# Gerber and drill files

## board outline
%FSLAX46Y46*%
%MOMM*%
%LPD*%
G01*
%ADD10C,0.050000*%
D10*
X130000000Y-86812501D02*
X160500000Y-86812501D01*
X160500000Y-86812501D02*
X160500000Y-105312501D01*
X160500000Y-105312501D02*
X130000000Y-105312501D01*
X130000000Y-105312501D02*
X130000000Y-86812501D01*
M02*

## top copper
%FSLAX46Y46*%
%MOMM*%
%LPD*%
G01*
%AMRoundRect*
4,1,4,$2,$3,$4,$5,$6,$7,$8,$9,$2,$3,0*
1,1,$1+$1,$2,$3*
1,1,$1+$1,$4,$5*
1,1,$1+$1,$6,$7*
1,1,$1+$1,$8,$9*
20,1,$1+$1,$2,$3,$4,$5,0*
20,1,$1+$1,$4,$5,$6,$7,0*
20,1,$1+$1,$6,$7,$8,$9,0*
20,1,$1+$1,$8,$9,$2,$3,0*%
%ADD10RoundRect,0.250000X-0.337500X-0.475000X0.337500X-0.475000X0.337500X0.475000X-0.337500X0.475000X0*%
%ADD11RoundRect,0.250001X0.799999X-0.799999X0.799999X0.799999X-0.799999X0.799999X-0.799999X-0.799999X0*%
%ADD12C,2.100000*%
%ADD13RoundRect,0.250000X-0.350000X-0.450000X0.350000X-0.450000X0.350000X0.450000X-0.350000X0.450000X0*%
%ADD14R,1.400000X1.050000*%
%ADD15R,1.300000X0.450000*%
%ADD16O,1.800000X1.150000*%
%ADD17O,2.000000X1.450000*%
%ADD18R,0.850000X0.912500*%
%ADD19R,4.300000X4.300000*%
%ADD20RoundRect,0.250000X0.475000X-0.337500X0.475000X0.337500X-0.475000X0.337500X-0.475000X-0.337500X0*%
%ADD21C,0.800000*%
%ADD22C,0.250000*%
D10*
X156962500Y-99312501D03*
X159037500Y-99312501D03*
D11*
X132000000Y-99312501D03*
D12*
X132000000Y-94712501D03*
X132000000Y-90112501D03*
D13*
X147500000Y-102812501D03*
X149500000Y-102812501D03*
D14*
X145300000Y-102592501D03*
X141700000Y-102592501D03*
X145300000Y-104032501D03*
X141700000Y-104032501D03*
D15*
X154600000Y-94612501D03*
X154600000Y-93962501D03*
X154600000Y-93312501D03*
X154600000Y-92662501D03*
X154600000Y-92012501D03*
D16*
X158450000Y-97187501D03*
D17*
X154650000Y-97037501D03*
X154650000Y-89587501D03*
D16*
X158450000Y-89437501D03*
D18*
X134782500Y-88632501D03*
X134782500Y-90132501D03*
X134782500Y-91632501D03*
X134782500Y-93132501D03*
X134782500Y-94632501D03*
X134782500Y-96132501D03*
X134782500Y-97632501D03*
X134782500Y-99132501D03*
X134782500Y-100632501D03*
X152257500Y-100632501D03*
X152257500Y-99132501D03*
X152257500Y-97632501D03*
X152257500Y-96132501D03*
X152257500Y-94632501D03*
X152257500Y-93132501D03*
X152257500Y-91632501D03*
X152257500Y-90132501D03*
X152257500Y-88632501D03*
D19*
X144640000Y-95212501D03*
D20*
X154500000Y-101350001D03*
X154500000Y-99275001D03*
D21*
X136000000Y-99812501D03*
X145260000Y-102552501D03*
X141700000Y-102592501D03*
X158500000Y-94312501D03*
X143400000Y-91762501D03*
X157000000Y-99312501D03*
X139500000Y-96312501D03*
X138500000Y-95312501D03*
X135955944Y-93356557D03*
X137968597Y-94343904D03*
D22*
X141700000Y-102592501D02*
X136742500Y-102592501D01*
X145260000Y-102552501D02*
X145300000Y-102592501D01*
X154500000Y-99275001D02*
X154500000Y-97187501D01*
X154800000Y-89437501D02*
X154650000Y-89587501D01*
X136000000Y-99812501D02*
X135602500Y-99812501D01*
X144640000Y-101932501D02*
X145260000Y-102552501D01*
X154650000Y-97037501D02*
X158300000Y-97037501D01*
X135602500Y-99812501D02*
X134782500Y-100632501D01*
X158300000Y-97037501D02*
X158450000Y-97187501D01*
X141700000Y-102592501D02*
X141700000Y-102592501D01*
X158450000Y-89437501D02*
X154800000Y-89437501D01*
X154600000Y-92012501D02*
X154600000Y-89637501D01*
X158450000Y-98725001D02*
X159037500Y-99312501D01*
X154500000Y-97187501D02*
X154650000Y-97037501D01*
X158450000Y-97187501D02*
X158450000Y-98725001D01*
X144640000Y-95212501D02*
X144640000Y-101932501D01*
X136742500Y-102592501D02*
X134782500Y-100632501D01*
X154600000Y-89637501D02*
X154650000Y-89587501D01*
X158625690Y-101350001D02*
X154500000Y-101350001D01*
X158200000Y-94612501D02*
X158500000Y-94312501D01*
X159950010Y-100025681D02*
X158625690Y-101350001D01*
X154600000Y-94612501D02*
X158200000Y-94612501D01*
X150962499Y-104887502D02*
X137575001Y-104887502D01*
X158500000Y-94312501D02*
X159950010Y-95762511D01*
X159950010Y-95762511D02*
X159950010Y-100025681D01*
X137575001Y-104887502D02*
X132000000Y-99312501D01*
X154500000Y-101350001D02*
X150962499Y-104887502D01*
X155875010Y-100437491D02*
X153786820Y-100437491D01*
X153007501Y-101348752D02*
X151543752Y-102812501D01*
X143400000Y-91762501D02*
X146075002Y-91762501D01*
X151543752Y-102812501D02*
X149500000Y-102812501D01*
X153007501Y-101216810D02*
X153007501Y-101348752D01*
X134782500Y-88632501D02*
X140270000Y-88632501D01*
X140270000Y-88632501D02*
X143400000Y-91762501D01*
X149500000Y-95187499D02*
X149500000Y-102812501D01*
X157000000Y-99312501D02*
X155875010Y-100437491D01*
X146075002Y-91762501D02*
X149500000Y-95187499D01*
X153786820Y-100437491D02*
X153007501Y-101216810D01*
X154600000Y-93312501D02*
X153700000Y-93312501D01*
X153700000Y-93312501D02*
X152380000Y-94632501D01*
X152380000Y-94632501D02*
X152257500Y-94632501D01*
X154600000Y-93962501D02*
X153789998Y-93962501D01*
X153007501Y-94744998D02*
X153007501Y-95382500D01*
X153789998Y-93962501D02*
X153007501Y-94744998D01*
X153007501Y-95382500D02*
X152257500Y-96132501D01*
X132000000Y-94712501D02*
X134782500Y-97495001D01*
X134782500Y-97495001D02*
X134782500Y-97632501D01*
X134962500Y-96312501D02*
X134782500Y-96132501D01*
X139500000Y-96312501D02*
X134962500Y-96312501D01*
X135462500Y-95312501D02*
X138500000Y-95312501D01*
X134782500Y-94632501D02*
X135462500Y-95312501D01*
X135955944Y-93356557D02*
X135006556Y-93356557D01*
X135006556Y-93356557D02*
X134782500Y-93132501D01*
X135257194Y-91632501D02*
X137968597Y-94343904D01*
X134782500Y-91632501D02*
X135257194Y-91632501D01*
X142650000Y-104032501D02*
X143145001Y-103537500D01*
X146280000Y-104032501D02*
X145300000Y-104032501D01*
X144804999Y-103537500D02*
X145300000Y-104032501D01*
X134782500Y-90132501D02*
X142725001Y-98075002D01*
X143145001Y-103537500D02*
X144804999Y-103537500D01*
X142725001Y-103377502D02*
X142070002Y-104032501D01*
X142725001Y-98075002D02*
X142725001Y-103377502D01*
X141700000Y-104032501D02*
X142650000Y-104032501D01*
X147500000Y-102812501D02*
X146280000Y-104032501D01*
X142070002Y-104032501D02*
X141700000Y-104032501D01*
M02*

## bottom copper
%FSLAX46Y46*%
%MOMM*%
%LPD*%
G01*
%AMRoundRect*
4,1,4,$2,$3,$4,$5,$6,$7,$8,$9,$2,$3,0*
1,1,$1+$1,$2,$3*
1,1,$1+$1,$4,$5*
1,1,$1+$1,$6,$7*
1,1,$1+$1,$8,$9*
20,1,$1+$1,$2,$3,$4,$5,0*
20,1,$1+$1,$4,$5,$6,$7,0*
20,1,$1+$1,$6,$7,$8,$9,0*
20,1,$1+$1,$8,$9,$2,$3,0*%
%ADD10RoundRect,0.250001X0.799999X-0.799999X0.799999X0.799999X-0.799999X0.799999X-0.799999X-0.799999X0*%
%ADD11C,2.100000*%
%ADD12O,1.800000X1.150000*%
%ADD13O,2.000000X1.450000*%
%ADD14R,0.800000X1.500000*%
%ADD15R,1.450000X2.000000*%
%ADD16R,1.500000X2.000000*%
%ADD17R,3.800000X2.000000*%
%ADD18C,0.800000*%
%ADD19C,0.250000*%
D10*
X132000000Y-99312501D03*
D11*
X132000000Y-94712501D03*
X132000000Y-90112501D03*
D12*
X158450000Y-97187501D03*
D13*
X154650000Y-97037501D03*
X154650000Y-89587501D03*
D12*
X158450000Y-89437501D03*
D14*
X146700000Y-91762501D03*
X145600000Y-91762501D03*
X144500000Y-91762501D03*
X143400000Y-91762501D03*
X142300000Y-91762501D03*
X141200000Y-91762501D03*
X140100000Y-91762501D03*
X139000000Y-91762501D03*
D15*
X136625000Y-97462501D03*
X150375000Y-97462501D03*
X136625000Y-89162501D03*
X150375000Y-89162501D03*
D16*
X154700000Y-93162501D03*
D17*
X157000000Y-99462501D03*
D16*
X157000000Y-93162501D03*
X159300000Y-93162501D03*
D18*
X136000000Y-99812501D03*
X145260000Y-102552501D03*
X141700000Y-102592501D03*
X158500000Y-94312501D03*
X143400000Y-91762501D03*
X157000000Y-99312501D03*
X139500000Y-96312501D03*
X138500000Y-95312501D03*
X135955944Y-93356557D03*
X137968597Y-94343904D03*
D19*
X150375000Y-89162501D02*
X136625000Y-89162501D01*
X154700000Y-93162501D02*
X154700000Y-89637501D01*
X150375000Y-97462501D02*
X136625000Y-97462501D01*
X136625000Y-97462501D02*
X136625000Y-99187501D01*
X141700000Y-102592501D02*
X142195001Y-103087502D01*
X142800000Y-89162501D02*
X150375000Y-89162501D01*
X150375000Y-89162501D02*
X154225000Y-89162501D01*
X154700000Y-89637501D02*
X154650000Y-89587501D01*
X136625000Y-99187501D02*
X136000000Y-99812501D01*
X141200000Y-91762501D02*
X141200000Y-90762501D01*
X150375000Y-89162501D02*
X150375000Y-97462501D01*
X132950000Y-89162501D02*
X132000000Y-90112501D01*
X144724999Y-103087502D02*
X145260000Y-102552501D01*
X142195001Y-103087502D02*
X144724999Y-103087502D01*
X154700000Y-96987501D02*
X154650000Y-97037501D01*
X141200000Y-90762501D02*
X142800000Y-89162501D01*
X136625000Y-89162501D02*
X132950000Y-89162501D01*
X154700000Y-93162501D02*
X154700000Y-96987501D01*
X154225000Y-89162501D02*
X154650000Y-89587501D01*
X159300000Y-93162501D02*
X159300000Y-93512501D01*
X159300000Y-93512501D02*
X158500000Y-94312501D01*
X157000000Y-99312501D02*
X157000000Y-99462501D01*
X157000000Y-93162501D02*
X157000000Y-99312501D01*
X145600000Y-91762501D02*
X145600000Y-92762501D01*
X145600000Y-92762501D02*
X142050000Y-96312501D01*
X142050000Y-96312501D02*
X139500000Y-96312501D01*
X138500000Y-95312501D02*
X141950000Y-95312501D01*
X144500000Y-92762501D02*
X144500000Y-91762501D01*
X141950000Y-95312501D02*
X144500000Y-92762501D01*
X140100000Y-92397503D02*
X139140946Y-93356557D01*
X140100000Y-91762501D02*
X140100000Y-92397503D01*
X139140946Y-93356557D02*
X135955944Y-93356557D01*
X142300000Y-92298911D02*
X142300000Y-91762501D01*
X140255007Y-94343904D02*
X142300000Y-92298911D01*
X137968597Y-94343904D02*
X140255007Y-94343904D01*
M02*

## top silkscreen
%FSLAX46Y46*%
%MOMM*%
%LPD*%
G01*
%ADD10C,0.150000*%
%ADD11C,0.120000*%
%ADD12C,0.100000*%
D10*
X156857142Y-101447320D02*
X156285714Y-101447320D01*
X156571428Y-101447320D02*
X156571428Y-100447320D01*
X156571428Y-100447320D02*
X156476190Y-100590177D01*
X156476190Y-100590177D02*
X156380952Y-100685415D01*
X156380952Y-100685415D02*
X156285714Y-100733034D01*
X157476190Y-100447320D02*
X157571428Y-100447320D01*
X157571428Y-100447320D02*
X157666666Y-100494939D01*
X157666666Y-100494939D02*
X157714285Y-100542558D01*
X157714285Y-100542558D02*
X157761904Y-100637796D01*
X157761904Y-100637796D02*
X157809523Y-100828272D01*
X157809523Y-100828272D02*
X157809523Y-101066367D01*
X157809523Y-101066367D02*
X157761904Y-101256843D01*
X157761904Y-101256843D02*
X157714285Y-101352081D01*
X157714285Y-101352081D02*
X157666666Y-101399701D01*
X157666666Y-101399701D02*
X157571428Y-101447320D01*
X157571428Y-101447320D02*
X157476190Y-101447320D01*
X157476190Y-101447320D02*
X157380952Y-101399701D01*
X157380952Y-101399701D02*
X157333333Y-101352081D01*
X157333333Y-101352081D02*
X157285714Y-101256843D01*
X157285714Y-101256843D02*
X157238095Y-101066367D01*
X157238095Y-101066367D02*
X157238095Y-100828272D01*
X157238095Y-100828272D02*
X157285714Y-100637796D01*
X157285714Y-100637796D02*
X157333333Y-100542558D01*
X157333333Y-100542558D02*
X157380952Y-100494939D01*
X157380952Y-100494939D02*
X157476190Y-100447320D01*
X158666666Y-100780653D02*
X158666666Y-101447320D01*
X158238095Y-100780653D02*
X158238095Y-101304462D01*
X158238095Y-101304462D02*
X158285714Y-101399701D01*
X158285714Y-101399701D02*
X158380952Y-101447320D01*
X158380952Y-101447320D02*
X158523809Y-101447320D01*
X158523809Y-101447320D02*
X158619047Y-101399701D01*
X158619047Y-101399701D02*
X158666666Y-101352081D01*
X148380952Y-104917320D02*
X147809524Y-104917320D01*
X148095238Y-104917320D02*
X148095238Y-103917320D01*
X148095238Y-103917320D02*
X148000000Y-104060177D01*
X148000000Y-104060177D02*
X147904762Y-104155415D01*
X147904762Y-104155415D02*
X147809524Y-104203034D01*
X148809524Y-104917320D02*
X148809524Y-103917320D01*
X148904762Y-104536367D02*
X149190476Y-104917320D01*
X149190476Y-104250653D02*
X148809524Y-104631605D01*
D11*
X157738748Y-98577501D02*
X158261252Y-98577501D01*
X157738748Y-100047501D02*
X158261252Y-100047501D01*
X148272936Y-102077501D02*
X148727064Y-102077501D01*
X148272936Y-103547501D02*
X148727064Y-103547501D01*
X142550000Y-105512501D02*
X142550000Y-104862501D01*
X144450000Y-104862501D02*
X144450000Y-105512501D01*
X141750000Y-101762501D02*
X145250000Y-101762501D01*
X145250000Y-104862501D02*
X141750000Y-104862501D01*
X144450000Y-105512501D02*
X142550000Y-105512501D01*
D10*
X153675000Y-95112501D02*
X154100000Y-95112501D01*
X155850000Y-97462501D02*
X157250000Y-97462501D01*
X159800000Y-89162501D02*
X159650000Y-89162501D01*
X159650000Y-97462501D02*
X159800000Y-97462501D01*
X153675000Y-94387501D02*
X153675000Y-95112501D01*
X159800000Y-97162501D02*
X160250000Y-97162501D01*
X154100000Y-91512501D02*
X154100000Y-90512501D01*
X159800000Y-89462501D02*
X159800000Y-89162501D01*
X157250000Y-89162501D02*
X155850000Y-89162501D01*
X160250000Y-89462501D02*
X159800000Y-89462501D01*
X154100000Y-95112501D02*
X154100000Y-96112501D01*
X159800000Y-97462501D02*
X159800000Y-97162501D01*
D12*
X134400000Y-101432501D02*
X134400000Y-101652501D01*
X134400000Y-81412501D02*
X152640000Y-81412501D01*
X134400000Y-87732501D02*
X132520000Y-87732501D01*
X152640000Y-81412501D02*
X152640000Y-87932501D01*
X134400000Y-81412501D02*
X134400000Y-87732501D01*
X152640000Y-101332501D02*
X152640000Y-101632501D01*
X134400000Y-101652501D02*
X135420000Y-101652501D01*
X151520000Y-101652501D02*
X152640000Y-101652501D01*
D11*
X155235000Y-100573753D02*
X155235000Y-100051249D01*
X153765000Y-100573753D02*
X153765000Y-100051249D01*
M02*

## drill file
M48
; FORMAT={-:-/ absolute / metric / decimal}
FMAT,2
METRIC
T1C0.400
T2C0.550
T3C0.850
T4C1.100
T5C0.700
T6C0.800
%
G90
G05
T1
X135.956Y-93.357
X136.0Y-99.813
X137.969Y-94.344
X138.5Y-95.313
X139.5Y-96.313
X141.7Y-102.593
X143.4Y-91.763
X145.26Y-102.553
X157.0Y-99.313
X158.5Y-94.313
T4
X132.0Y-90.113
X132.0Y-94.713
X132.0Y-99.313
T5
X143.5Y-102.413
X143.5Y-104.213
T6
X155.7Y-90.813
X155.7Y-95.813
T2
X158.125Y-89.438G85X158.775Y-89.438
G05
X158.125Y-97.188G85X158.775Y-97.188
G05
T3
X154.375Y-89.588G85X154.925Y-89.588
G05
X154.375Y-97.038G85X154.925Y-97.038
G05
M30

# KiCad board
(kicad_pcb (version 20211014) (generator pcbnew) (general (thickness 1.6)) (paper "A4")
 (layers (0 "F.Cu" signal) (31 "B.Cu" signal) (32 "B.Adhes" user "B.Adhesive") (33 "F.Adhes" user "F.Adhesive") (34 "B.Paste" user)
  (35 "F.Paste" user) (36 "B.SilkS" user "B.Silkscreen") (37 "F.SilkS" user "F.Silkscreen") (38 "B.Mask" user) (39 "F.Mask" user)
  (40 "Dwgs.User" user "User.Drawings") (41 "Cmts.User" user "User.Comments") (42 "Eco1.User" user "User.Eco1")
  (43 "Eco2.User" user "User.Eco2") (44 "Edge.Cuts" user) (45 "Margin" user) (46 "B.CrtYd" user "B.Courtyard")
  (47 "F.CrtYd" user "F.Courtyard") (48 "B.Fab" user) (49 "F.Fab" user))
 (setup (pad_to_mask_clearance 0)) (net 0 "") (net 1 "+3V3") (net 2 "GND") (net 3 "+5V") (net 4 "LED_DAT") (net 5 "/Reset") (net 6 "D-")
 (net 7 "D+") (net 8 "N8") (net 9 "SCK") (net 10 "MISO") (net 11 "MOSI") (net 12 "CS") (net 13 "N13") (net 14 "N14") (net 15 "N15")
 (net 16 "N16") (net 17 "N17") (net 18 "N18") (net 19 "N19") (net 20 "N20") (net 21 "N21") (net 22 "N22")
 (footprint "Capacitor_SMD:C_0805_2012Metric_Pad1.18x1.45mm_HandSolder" (layer "F.Cu") (at 158 99.312501)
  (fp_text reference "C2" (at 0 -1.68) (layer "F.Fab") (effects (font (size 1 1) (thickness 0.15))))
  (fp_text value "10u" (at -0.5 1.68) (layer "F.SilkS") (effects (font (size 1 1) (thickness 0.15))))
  (fp_line (start -0.261252 -0.735) (end 0.261252 -0.735) (layer "F.SilkS") (width 0.12))
  (fp_line (start -0.261252 0.735) (end 0.261252 0.735) (layer "F.SilkS") (width 0.12))
  (pad "1" smd roundrect locked (at -1.0375 0) (size 1.175 1.45) (layers "F.Cu" "F.Paste" "F.Mask") (roundrect_rratio 0.2127659574)
   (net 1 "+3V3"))
  (pad "2" smd roundrect locked (at 1.0375 0) (size 1.175 1.45) (layers "F.Cu" "F.Paste" "F.Mask") (roundrect_rratio 0.2127659574)
   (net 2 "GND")))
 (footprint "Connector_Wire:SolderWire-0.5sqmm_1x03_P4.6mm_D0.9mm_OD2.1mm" (layer "F.Cu") (at 132 99.312501 90)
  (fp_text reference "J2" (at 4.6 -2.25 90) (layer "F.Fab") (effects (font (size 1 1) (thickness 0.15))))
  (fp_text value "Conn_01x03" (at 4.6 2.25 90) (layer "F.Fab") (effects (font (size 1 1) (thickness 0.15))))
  (pad "1" thru_hole roundrect locked (at 0 0 90) (size 2.1 2.1) (drill 1.1) (layers *.Cu *.Mask) (roundrect_rratio 0.1190480952)
   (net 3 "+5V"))
  (pad "2" thru_hole circle locked (at 4.6 0 90) (size 2.1 2.1) (drill 1.1) (layers *.Cu *.Mask) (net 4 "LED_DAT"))
  (pad "3" thru_hole circle locked (at 9.2 0 90) (size 2.1 2.1) (drill 1.1) (layers *.Cu *.Mask) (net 2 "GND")))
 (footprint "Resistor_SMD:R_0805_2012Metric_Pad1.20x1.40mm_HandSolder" (layer "F.Cu") (at 148.5 102.812501)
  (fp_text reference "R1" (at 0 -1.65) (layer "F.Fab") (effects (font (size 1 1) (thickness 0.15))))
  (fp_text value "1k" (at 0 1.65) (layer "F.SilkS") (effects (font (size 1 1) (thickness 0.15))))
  (fp_line (start -0.227064 -0.735) (end 0.227064 -0.735) (layer "F.SilkS") (width 0.12))
  (fp_line (start -0.227064 0.735) (end 0.227064 0.735) (layer "F.SilkS") (width 0.12))
  (pad "1" smd roundrect locked (at -1 0) (size 1.2 1.4) (layers "F.Cu" "F.Paste" "F.Mask") (roundrect_rratio 0.2083333333) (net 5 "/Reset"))
  (pad "2" smd roundrect locked (at 1 0) (size 1.2 1.4) (layers "F.Cu" "F.Paste" "F.Mask") (roundrect_rratio 0.2083333333) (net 1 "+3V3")))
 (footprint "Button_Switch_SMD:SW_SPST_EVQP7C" (layer "F.Cu") (at 143.5 103.312501)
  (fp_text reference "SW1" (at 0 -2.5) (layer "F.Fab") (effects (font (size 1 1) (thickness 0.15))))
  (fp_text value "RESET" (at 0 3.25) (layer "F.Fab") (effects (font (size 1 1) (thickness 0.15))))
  (fp_line (start -0.95 2.2) (end -0.95 1.55) (layer "F.SilkS") (width 0.12))
  (fp_line (start 0.95 1.55) (end 0.95 2.2) (layer "F.SilkS") (width 0.12))
  (fp_line (start -1.75 -1.55) (end 1.75 -1.55) (layer "F.SilkS") (width 0.12))
  (fp_line (start 1.75 1.55) (end -1.75 1.55) (layer "F.SilkS") (width 0.12))
  (fp_line (start 0.95 2.2) (end -0.95 2.2) (layer "F.SilkS") (width 0.12))
  (pad "" np_thru_hole circle locked (at 0 0.9) (size 0.7 0.7) (drill 0.7) (layers *.Cu *.Mask))
  (pad "" np_thru_hole circle locked (at 0 -0.9) (size 0.7 0.7) (drill 0.7) (layers *.Cu *.Mask))
  (pad "1" smd rect locked (at 1.8 -0.72) (size 1.4 1.05) (layers "F.Cu" "F.Paste" "F.Mask") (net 2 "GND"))
  (pad "1" smd rect locked (at -1.8 -0.72) (size 1.4 1.05) (layers "F.Cu" "F.Paste" "F.Mask") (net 2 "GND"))
  (pad "2" smd rect locked (at 1.8 0.72) (size 1.4 1.05) (layers "F.Cu" "F.Paste" "F.Mask") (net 5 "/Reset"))
  (pad "2" smd rect locked (at -1.8 0.72) (size 1.4 1.05) (layers "F.Cu" "F.Paste" "F.Mask") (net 5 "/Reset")))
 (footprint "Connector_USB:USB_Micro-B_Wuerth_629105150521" (layer "F.Cu") (at 156.5 93.312501 90)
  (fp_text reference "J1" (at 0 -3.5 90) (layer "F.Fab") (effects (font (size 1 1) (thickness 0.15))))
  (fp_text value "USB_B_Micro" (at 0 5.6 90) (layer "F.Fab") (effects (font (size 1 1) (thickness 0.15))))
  (fp_line (start -1.8 -2.825) (end -1.8 -2.4) (layer "F.SilkS") (width 0.15))
  (fp_line (start -4.15 -0.65) (end -4.15 0.75) (layer "F.SilkS") (width 0.15))
  (fp_line (start 4.15 3.3) (end 4.15 3.15) (layer "F.SilkS") (width 0.15))
  (fp_line (start -4.15 3.15) (end -4.15 3.3) (layer "F.SilkS") (width 0.15))
  (fp_line (start -1.075 -2.825) (end -1.8 -2.825) (layer "F.SilkS") (width 0.15))
  (fp_line (start -3.85 3.3) (end -3.85 3.75) (layer "F.SilkS") (width 0.15))
  (fp_line (start 1.8 -2.4) (end 2.8 -2.4) (layer "F.SilkS") (width 0.15))
  (fp_line (start 3.85 3.3) (end 4.15 3.3) (layer "F.SilkS") (width 0.15))
  (fp_line (start 4.15 0.75) (end 4.15 -0.65) (layer "F.SilkS") (width 0.15))
  (fp_line (start 3.85 3.75) (end 3.85 3.3) (layer "F.SilkS") (width 0.15))
  (fp_line (start -1.8 -2.4) (end -2.8 -2.4) (layer "F.SilkS") (width 0.15))
  (fp_line (start -4.15 3.3) (end -3.85 3.3) (layer "F.SilkS") (width 0.15))
  (pad "" np_thru_hole oval locked (at 2.5 -0.8 90) (size 0.8 0.8) (drill 0.8) (layers *.Cu *.Mask))
  (pad "" np_thru_hole oval locked (at -2.5 -0.8 90) (size 0.8 0.8) (drill 0.8) (layers *.Cu *.Mask))
  (pad "1" smd rect locked (at -1.3 -1.9 90) (size 0.45 1.3) (layers "F.Cu" "F.Paste" "F.Mask") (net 3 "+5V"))
  (pad "2" smd rect locked (at -0.65 -1.9 90) (size 0.45 1.3) (layers "F.Cu" "F.Paste" "F.Mask") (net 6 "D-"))
  (pad "3" smd rect locked (at 0 -1.9 90) (size 0.45 1.3) (layers "F.Cu" "F.Paste" "F.Mask") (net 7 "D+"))
  (pad "4" smd rect locked (at 0.65 -1.9 90) (size 0.45 1.3) (layers "F.Cu" "F.Paste" "F.Mask") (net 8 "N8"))
  (pad "5" smd rect locked (at 1.3 -1.9 90) (size 0.45 1.3) (layers "F.Cu" "F.Paste" "F.Mask") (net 2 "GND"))
  (pad "6" thru_hole oval locked (at -3.875 1.95 90) (size 1.15 1.8) (drill oval 0.55 1.2) (layers *.Cu *.Mask) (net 2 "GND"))
  (pad "6" thru_hole oval locked (at -3.725 -1.85 90) (size 1.45 2) (drill oval 0.85 1.4) (layers *.Cu *.Mask) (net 2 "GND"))
  (pad "6" thru_hole oval locked (at 3.725 -1.85 90) (size 1.45 2) (drill oval 0.85 1.4) (layers *.Cu *.Mask) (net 2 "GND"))
  (pad "6" thru_hole oval locked (at 3.875 1.95 90) (size 1.15 1.8) (drill oval 0.55 1.2) (layers *.Cu *.Mask) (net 2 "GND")))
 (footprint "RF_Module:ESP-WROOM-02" (layer "F.Cu") (at 143.52 94.632501)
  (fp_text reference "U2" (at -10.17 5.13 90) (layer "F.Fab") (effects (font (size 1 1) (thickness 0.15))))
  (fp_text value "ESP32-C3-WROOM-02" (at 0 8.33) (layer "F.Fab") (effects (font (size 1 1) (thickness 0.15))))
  (fp_line (start -9.12 6.8) (end -9.12 7.02) (layer "F.SilkS") (width 0.1))
  (fp_line (start -9.12 -13.22) (end 9.12 -13.22) (layer "F.SilkS") (width 0.1))
  (fp_line (start -9.12 -6.9) (end -11 -6.9) (layer "F.SilkS") (width 0.1))
  (fp_line (start 9.12 -13.22) (end 9.12 -6.7) (layer "F.SilkS") (width 0.1))
  (fp_line (start -9.12 -13.22) (end -9.12 -6.9) (layer "F.SilkS") (width 0.1))
  (fp_line (start 9.12 6.7) (end 9.12 7) (layer "F.SilkS") (width 0.1))
  (fp_line (start -9.12 7.02) (end -8.1 7.02) (layer "F.SilkS") (width 0.1))
  (fp_line (start 8 7.02) (end 9.12 7.02) (layer "F.SilkS") (width 0.1))
  (pad "1" smd rect locked (at -8.7375 -6) (size 0.85 0.9125) (layers "F.Cu" "F.Paste" "F.Mask") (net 1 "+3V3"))
  (pad "2" smd rect locked (at -8.7375 -4.5) (size 0.85 0.9125) (layers "F.Cu" "F.Paste" "F.Mask") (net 5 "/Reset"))
  (pad "3" smd rect locked (at -8.7375 -3) (size 0.85 0.9125) (layers "F.Cu" "F.Paste" "F.Mask") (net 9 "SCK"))
  (pad "4" smd rect locked (at -8.7375 -1.5) (size 0.85 0.9125) (layers "F.Cu" "F.Paste" "F.Mask") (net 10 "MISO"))
  (pad "5" smd rect locked (at -8.7375 0) (size 0.85 0.9125) (layers "F.Cu" "F.Paste" "F.Mask") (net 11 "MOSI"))
  (pad "6" smd rect locked (at -8.7375 1.5) (size 0.85 0.9125) (layers "F.Cu" "F.Paste" "F.Mask") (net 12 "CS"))
  (pad "7" smd rect locked (at -8.7375 3) (size 0.85 0.9125) (layers "F.Cu" "F.Paste" "F.Mask") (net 4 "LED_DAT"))
  (pad "8" smd rect locked (at -8.7375 4.5) (size 0.85 0.9125) (layers "F.Cu" "F.Paste" "F.Mask") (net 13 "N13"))
  (pad "9" smd rect locked (at -8.7375 6) (size 0.85 0.9125) (layers "F.Cu" "F.Paste" "F.Mask") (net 2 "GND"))
  (pad "10" smd rect locked (at 8.7375 6) (size 0.85 0.9125) (layers "F.Cu" "F.Paste" "F.Mask") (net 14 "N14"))
  (pad "11" smd rect locked (at 8.7375 4.5) (size 0.85 0.9125) (layers "F.Cu" "F.Paste" "F.Mask") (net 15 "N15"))
  (pad "12" smd rect locked (at 8.7375 3) (size 0.85 0.9125) (layers "F.Cu" "F.Paste" "F.Mask") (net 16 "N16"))
  (pad "13" smd rect locked (at 8.7375 1.5) (size 0.85 0.9125) (layers "F.Cu" "F.Paste" "F.Mask") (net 6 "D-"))
  (pad "14" smd rect locked (at 8.7375 0) (size 0.85 0.9125) (layers "F.Cu" "F.Paste" "F.Mask") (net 7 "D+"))
  (pad "15" smd rect locked (at 8.7375 -1.5) (size 0.85 0.9125) (layers "F.Cu" "F.Paste" "F.Mask") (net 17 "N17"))
  (pad "16" smd rect locked (at 8.7375 -3) (size 0.85 0.9125) (layers "F.Cu" "F.Paste" "F.Mask") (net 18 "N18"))
  (pad "17" smd rect locked (at 8.7375 -4.5) (size 0.85 0.9125) (layers "F.Cu" "F.Paste" "F.Mask") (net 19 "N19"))
  (pad "18" smd rect locked (at 8.7375 -6) (size 0.85 0.9125) (layers "F.Cu" "F.Paste" "F.Mask") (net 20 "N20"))
  (pad "19" smd rect locked (at 1.12 0.58) (size 4.3 4.3) (layers "F.Cu" "F.Paste" "F.Mask") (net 2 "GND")))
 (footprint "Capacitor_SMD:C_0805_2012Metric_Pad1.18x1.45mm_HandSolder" (layer "F.Cu") (at 154.5 100.312501 90)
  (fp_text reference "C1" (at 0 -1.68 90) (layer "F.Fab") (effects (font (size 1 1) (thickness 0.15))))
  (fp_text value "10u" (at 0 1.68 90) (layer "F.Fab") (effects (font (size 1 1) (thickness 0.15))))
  (fp_line (start -0.261252 0.735) (end 0.261252 0.735) (layer "F.SilkS") (width 0.12))
  (fp_line (start -0.261252 -0.735) (end 0.261252 -0.735) (layer "F.SilkS") (width 0.12))
  (pad "1" smd roundrect locked (at -1.0375 0 90) (size 1.175 1.45) (layers "F.Cu" "F.Paste" "F.Mask") (roundrect_rratio 0.2127659574)
   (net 3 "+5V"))
  (pad "2" smd roundrect locked (at 1.0375 0 90) (size 1.175 1.45) (layers "F.Cu" "F.Paste" "F.Mask") (roundrect_rratio 0.2127659574)
   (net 2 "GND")))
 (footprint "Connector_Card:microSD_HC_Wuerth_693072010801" (layer "B.Cu") (at 143.5 93.312501 180)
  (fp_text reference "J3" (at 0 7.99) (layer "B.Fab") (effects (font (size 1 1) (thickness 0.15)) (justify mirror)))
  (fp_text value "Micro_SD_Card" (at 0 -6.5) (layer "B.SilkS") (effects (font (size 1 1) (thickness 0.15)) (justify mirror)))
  (pad "1" smd rect locked (at -3.2 1.55 180) (size 0.8 1.5) (layers "B.Cu" "B.Paste" "B.Mask") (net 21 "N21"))
  (pad "2" smd rect locked (at -2.1 1.55 180) (size 0.8 1.5) (layers "B.Cu" "B.Paste" "B.Mask") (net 12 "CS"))
  (pad "3" smd rect locked (at -1 1.55 180) (size 0.8 1.5) (layers "B.Cu" "B.Paste" "B.Mask") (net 11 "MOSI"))
  (pad "4" smd rect locked (at 0.1 1.55 180) (size 0.8 1.5) (layers "B.Cu" "B.Paste" "B.Mask") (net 1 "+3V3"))
  (pad "5" smd rect locked (at 1.2 1.55 180) (size 0.8 1.5) (layers "B.Cu" "B.Paste" "B.Mask") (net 9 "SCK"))
  (pad "6" smd rect locked (at 2.3 1.55 180) (size 0.8 1.5) (layers "B.Cu" "B.Paste" "B.Mask") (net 2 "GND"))
  (pad "7" smd rect locked (at 3.4 1.55 180) (size 0.8 1.5) (layers "B.Cu" "B.Paste" "B.Mask") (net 10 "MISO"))
  (pad "8" smd rect locked (at 4.5 1.55 180) (size 0.8 1.5) (layers "B.Cu" "B.Paste" "B.Mask") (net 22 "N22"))
  (pad "9" smd rect locked (at 6.875 -4.15 180) (size 1.45 2) (layers "B.Cu" "B.Paste" "B.Mask") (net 2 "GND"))
  (pad "9" smd rect locked (at -6.875 -4.15 180) (size 1.45 2) (layers "B.Cu" "B.Paste" "B.Mask") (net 2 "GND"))
  (pad "9" smd rect locked (at 6.875 4.15 180) (size 1.45 2) (layers "B.Cu" "B.Paste" "B.Mask") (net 2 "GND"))
  (pad "9" smd rect locked (at -6.875 4.15 180) (size 1.45 2) (layers "B.Cu" "B.Paste" "B.Mask") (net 2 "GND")))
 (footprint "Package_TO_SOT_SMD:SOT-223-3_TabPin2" (layer "B.Cu") (at 157 96.312501 -90)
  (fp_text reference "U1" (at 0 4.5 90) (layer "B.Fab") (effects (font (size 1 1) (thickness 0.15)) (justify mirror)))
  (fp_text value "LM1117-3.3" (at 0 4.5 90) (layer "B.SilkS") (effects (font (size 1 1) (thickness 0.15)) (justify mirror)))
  (pad "1" smd rect locked (at -3.15 2.3 270) (size 2 1.5) (layers "B.Cu" "B.Paste" "B.Mask") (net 2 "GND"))
  (pad "2" smd rect locked (at 3.15 0 270) (size 2 3.8) (layers "B.Cu" "B.Paste" "B.Mask") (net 1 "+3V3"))
  (pad "2" smd rect locked (at -3.15 0 270) (size 2 1.5) (layers "B.Cu" "B.Paste" "B.Mask") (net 1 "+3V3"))
  (pad "3" smd rect locked (at -3.15 -2.3 270) (size 2 1.5) (layers "B.Cu" "B.Paste" "B.Mask") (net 3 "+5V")))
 (gr_line (start 130 86.812501) (end 160.5 86.812501) (layer "Edge.Cuts") (width 0.05))
 (gr_line (start 160.5 86.812501) (end 160.5 105.312501) (layer "Edge.Cuts") (width 0.05))
 (gr_line (start 160.5 105.312501) (end 130 105.312501) (layer "Edge.Cuts") (width 0.05))
 (gr_line (start 130 105.312501) (end 130 86.812501) (layer "Edge.Cuts") (width 0.05))
 (segment (start 141.7 102.592501) (end 136.7425 102.592501) (width 0.25) (layer "F.Cu") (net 2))
 (segment (start 145.26 102.552501) (end 145.3 102.592501) (width 0.25) (layer "F.Cu") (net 2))
 (segment (start 154.5 99.275001) (end 154.5 97.187501) (width 0.25) (layer "F.Cu") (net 2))
 (segment (start 154.8 89.437501) (end 154.65 89.587501) (width 0.25) (layer "F.Cu") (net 2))
 (segment (start 136 99.812501) (end 135.6025 99.812501) (width 0.25) (layer "F.Cu") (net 2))
 (segment (start 144.64 101.932501) (end 145.26 102.552501) (width 0.25) (layer "F.Cu") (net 2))
 (segment (start 154.65 97.037501) (end 158.3 97.037501) (width 0.25) (layer "F.Cu") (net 2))
 (segment (start 135.6025 99.812501) (end 134.7825 100.632501) (width 0.25) (layer "F.Cu") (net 2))
 (segment (start 158.3 97.037501) (end 158.45 97.187501) (width 0.25) (layer "F.Cu") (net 2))
 (segment (start 141.7 102.592501) (end 141.7 102.592501) (width 0.25) (layer "F.Cu") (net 2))
 (segment (start 158.45 89.437501) (end 154.8 89.437501) (width 0.25) (layer "F.Cu") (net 2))
 (segment (start 154.6 92.012501) (end 154.6 89.637501) (width 0.25) (layer "F.Cu") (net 2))
 (segment (start 158.45 98.725001) (end 159.0375 99.312501) (width 0.25) (layer "F.Cu") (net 2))
 (segment (start 154.5 97.187501) (end 154.65 97.037501) (width 0.25) (layer "F.Cu") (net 2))
 (segment (start 158.45 97.187501) (end 158.45 98.725001) (width 0.25) (layer "F.Cu") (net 2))
 (segment (start 144.64 95.212501) (end 144.64 101.932501) (width 0.25) (layer "F.Cu") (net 2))
 (segment (start 136.7425 102.592501) (end 134.7825 100.632501) (width 0.25) (layer "F.Cu") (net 2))
 (segment (start 154.6 89.637501) (end 154.65 89.587501) (width 0.25) (layer "F.Cu") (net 2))
 (via (at 136 99.812501) (size 0.8) (drill 0.4) (layers "F.Cu" "B.Cu") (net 2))
 (via (at 145.26 102.552501) (size 0.8) (drill 0.4) (layers "F.Cu" "B.Cu") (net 2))
 (via (at 141.7 102.592501) (size 0.8) (drill 0.4) (layers "F.Cu" "B.Cu") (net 2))
 (segment (start 150.375 89.162501) (end 136.625 89.162501) (width 0.25) (layer "B.Cu") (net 2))
 (segment (start 154.7 93.162501) (end 154.7 89.637501) (width 0.25) (layer "B.Cu") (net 2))
 (segment (start 150.375 97.462501) (end 136.625 97.462501) (width 0.25) (layer "B.Cu") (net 2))
 (segment (start 136.625 97.462501) (end 136.625 99.187501) (width 0.25) (layer "B.Cu") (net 2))
 (segment (start 141.7 102.592501) (end 142.195001 103.087502) (width 0.25) (layer "B.Cu") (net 2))
 (segment (start 142.8 89.162501) (end 150.375 89.162501) (width 0.25) (layer "B.Cu") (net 2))
 (segment (start 150.375 89.162501) (end 154.225 89.162501) (width 0.25) (layer "B.Cu") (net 2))
 (segment (start 154.7 89.637501) (end 154.65 89.587501) (width 0.25) (layer "B.Cu") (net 2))
 (segment (start 136.625 99.187501) (end 136 99.812501) (width 0.25) (layer "B.Cu") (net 2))
 (segment (start 141.2 91.762501) (end 141.2 90.762501) (width 0.25) (layer "B.Cu") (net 2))
 (segment (start 150.375 89.162501) (end 150.375 97.462501) (width 0.25) (layer "B.Cu") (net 2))
 (segment (start 132.95 89.162501) (end 132 90.112501) (width 0.25) (layer "B.Cu") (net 2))
 (segment (start 144.724999 103.087502) (end 145.26 102.552501) (width 0.25) (layer "B.Cu") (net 2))
 (segment (start 142.195001 103.087502) (end 144.724999 103.087502) (width 0.25) (layer "B.Cu") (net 2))
 (segment (start 154.7 96.987501) (end 154.65 97.037501) (width 0.25) (layer "B.Cu") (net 2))
 (segment (start 141.2 90.762501) (end 142.8 89.162501) (width 0.25) (layer "B.Cu") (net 2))
 (segment (start 136.625 89.162501) (end 132.95 89.162501) (width 0.25) (layer "B.Cu") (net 2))
 (segment (start 154.7 93.162501) (end 154.7 96.987501) (width 0.25) (layer "B.Cu") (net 2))
 (segment (start 154.225 89.162501) (end 154.65 89.587501) (width 0.25) (layer "B.Cu") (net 2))
 (segment (start 158.62569 101.350001) (end 154.5 101.350001) (width 0.25) (layer "F.Cu") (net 3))
 (segment (start 158.2 94.612501) (end 158.5 94.312501) (width 0.25) (layer "F.Cu") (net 3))
 (segment (start 159.95001 100.025681) (end 158.62569 101.350001) (width 0.25) (layer "F.Cu") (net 3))
 (segment (start 154.6 94.612501) (end 158.2 94.612501) (width 0.25) (layer "F.Cu") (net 3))
 (segment (start 150.962499 104.887502) (end 137.575001 104.887502) (width 0.25) (layer "F.Cu") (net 3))
 (segment (start 158.5 94.312501) (end 159.95001 95.762511) (width 0.25) (layer "F.Cu") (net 3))
 (segment (start 159.95001 95.762511) (end 159.95001 100.025681) (width 0.25) (layer "F.Cu") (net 3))
 (segment (start 137.575001 104.887502) (end 132 99.312501) (width 0.25) (layer "F.Cu") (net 3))
 (segment (start 154.5 101.350001) (end 150.962499 104.887502) (width 0.25) (layer "F.Cu") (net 3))
 (via (at 158.5 94.312501) (size 0.8) (drill 0.4) (layers "F.Cu" "B.Cu") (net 3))
 (segment (start 159.3 93.162501) (end 159.3 93.512501) (width 0.25) (layer "B.Cu") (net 3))
 (segment (start 159.3 93.512501) (end 158.5 94.312501) (width 0.25) (layer "B.Cu") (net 3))
 (segment (start 155.87501 100.437491) (end 153.78682 100.437491) (width 0.25) (layer "F.Cu") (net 1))
 (segment (start 153.007501 101.348752) (end 151.543752 102.812501) (width 0.25) (layer "F.Cu") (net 1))
 (segment (start 143.4 91.762501) (end 146.075002 91.762501) (width 0.25) (layer "F.Cu") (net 1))
 (segment (start 151.543752 102.812501) (end 149.5 102.812501) (width 0.25) (layer "F.Cu") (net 1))
 (segment (start 153.007501 101.21681) (end 153.007501 101.348752) (width 0.25) (layer "F.Cu") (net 1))
 (segment (start 134.7825 88.632501) (end 140.27 88.632501) (width 0.25) (layer "F.Cu") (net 1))
 (segment (start 140.27 88.632501) (end 143.4 91.762501) (width 0.25) (layer "F.Cu") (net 1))
 (segment (start 149.5 95.187499) (end 149.5 102.812501) (width 0.25) (layer "F.Cu") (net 1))
 (segment (start 157 99.312501) (end 155.87501 100.437491) (width 0.25) (layer "F.Cu") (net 1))
 (segment (start 146.075002 91.762501) (end 149.5 95.187499) (width 0.25) (layer "F.Cu") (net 1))
 (segment (start 153.78682 100.437491) (end 153.007501 101.21681) (width 0.25) (layer "F.Cu") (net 1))
 (via (at 143.4 91.762501) (size 0.8) (drill 0.4) (layers "F.Cu" "B.Cu") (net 1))
 (via (at 157 99.312501) (size 0.8) (drill 0.4) (layers "F.Cu" "B.Cu") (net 1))
 (segment (start 157 99.312501) (end 157 99.462501) (width 0.25) (layer "B.Cu") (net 1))
 (segment (start 157 93.162501) (end 157 99.312501) (width 0.25) (layer "B.Cu") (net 1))
 (segment (start 154.6 93.312501) (end 153.7 93.312501) (width 0.25) (layer "F.Cu") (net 7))
 (segment (start 153.7 93.312501) (end 152.38 94.632501) (width 0.25) (layer "F.Cu") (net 7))
 (segment (start 152.38 94.632501) (end 152.2575 94.632501) (width 0.25) (layer "F.Cu") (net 7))
 (segment (start 154.6 93.962501) (end 153.789998 93.962501) (width 0.25) (layer "F.Cu") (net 6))
 (segment (start 153.007501 94.744998) (end 153.007501 95.3825) (width 0.25) (layer "F.Cu") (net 6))
 (segment (start 153.789998 93.962501) (end 153.007501 94.744998) (width 0.25) (layer "F.Cu") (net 6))
 (segment (start 153.007501 95.3825) (end 152.2575 96.132501) (width 0.25) (layer "F.Cu") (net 6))
 (segment (start 132 94.712501) (end 134.7825 97.495001) (width 0.25) (layer "F.Cu") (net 4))
 (segment (start 134.7825 97.495001) (end 134.7825 97.632501) (width 0.25) (layer "F.Cu") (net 4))
 (segment (start 134.9625 96.312501) (end 134.7825 96.132501) (width 0.25) (layer "F.Cu") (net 12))
 (segment (start 139.5 96.312501) (end 134.9625 96.312501) (width 0.25) (layer "F.Cu") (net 12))
 (via (at 139.5 96.312501) (size 0.8) (drill 0.4) (layers "F.Cu" "B.Cu") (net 12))
 (segment (start 145.6 91.762501) (end 145.6 92.762501) (width 0.25) (layer "B.Cu") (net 12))
 (segment (start 145.6 92.762501) (end 142.05 96.312501) (width 0.25) (layer "B.Cu") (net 12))
 (segment (start 142.05 96.312501) (end 139.5 96.312501) (width 0.25) (layer "B.Cu") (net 12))
 (segment (start 135.4625 95.312501) (end 138.5 95.312501) (width 0.25) (layer "F.Cu") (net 11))
 (segment (start 134.7825 94.632501) (end 135.4625 95.312501) (width 0.25) (layer "F.Cu") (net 11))
 (via (at 138.5 95.312501) (size 0.8) (drill 0.4) (layers "F.Cu" "B.Cu") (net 11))
 (segment (start 138.5 95.312501) (end 141.95 95.312501) (width 0.25) (layer "B.Cu") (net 11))
 (segment (start 144.5 92.762501) (end 144.5 91.762501) (width 0.25) (layer "B.Cu") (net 11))
 (segment (start 141.95 95.312501) (end 144.5 92.762501) (width 0.25) (layer "B.Cu") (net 11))
 (segment (start 135.955944 93.356557) (end 135.006556 93.356557) (width 0.25) (layer "F.Cu") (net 10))
 (segment (start 135.006556 93.356557) (end 134.7825 93.132501) (width 0.25) (layer "F.Cu") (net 10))
 (via (at 135.955944 93.356557) (size 0.8) (drill 0.4) (layers "F.Cu" "B.Cu") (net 10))
 (segment (start 140.1 92.397503) (end 139.140946 93.356557) (width 0.25) (layer "B.Cu") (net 10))
 (segment (start 140.1 91.762501) (end 140.1 92.397503) (width 0.25) (layer "B.Cu") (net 10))
 (segment (start 139.140946 93.356557) (end 135.955944 93.356557) (width 0.25) (layer "B.Cu") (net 10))
 (segment (start 135.257194 91.632501) (end 137.968597 94.343904) (width 0.25) (layer "F.Cu") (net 9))
 (segment (start 134.7825 91.632501) (end 135.257194 91.632501) (width 0.25) (layer "F.Cu") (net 9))
 (via (at 137.968597 94.343904) (size 0.8) (drill 0.4) (layers "F.Cu" "B.Cu") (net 9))
 (segment (start 142.3 92.298911) (end 142.3 91.762501) (width 0.25) (layer "B.Cu") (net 9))
 (segment (start 140.255007 94.343904) (end 142.3 92.298911) (width 0.25) (layer "B.Cu") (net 9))
 (segment (start 137.968597 94.343904) (end 140.255007 94.343904) (width 0.25) (layer "B.Cu") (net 9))
 (segment (start 142.65 104.032501) (end 143.145001 103.5375) (width 0.25) (layer "F.Cu") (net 5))
 (segment (start 146.28 104.032501) (end 145.3 104.032501) (width 0.25) (layer "F.Cu") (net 5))
 (segment (start 144.804999 103.5375) (end 145.3 104.032501) (width 0.25) (layer "F.Cu") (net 5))
 (segment (start 134.7825 90.132501) (end 142.725001 98.075002) (width 0.25) (layer "F.Cu") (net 5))
 (segment (start 143.145001 103.5375) (end 144.804999 103.5375) (width 0.25) (layer "F.Cu") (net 5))
 (segment (start 142.725001 103.377502) (end 142.070002 104.032501) (width 0.25) (layer "F.Cu") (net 5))
 (segment (start 142.725001 98.075002) (end 142.725001 103.377502) (width 0.25) (layer "F.Cu") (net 5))
 (segment (start 141.7 104.032501) (end 142.65 104.032501) (width 0.25) (layer "F.Cu") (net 5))
 (segment (start 147.5 102.812501) (end 146.28 104.032501) (width 0.25) (layer "F.Cu") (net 5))
 (segment (start 142.070002 104.032501) (end 141.7 104.032501) (width 0.25) (layer "F.Cu") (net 5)))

